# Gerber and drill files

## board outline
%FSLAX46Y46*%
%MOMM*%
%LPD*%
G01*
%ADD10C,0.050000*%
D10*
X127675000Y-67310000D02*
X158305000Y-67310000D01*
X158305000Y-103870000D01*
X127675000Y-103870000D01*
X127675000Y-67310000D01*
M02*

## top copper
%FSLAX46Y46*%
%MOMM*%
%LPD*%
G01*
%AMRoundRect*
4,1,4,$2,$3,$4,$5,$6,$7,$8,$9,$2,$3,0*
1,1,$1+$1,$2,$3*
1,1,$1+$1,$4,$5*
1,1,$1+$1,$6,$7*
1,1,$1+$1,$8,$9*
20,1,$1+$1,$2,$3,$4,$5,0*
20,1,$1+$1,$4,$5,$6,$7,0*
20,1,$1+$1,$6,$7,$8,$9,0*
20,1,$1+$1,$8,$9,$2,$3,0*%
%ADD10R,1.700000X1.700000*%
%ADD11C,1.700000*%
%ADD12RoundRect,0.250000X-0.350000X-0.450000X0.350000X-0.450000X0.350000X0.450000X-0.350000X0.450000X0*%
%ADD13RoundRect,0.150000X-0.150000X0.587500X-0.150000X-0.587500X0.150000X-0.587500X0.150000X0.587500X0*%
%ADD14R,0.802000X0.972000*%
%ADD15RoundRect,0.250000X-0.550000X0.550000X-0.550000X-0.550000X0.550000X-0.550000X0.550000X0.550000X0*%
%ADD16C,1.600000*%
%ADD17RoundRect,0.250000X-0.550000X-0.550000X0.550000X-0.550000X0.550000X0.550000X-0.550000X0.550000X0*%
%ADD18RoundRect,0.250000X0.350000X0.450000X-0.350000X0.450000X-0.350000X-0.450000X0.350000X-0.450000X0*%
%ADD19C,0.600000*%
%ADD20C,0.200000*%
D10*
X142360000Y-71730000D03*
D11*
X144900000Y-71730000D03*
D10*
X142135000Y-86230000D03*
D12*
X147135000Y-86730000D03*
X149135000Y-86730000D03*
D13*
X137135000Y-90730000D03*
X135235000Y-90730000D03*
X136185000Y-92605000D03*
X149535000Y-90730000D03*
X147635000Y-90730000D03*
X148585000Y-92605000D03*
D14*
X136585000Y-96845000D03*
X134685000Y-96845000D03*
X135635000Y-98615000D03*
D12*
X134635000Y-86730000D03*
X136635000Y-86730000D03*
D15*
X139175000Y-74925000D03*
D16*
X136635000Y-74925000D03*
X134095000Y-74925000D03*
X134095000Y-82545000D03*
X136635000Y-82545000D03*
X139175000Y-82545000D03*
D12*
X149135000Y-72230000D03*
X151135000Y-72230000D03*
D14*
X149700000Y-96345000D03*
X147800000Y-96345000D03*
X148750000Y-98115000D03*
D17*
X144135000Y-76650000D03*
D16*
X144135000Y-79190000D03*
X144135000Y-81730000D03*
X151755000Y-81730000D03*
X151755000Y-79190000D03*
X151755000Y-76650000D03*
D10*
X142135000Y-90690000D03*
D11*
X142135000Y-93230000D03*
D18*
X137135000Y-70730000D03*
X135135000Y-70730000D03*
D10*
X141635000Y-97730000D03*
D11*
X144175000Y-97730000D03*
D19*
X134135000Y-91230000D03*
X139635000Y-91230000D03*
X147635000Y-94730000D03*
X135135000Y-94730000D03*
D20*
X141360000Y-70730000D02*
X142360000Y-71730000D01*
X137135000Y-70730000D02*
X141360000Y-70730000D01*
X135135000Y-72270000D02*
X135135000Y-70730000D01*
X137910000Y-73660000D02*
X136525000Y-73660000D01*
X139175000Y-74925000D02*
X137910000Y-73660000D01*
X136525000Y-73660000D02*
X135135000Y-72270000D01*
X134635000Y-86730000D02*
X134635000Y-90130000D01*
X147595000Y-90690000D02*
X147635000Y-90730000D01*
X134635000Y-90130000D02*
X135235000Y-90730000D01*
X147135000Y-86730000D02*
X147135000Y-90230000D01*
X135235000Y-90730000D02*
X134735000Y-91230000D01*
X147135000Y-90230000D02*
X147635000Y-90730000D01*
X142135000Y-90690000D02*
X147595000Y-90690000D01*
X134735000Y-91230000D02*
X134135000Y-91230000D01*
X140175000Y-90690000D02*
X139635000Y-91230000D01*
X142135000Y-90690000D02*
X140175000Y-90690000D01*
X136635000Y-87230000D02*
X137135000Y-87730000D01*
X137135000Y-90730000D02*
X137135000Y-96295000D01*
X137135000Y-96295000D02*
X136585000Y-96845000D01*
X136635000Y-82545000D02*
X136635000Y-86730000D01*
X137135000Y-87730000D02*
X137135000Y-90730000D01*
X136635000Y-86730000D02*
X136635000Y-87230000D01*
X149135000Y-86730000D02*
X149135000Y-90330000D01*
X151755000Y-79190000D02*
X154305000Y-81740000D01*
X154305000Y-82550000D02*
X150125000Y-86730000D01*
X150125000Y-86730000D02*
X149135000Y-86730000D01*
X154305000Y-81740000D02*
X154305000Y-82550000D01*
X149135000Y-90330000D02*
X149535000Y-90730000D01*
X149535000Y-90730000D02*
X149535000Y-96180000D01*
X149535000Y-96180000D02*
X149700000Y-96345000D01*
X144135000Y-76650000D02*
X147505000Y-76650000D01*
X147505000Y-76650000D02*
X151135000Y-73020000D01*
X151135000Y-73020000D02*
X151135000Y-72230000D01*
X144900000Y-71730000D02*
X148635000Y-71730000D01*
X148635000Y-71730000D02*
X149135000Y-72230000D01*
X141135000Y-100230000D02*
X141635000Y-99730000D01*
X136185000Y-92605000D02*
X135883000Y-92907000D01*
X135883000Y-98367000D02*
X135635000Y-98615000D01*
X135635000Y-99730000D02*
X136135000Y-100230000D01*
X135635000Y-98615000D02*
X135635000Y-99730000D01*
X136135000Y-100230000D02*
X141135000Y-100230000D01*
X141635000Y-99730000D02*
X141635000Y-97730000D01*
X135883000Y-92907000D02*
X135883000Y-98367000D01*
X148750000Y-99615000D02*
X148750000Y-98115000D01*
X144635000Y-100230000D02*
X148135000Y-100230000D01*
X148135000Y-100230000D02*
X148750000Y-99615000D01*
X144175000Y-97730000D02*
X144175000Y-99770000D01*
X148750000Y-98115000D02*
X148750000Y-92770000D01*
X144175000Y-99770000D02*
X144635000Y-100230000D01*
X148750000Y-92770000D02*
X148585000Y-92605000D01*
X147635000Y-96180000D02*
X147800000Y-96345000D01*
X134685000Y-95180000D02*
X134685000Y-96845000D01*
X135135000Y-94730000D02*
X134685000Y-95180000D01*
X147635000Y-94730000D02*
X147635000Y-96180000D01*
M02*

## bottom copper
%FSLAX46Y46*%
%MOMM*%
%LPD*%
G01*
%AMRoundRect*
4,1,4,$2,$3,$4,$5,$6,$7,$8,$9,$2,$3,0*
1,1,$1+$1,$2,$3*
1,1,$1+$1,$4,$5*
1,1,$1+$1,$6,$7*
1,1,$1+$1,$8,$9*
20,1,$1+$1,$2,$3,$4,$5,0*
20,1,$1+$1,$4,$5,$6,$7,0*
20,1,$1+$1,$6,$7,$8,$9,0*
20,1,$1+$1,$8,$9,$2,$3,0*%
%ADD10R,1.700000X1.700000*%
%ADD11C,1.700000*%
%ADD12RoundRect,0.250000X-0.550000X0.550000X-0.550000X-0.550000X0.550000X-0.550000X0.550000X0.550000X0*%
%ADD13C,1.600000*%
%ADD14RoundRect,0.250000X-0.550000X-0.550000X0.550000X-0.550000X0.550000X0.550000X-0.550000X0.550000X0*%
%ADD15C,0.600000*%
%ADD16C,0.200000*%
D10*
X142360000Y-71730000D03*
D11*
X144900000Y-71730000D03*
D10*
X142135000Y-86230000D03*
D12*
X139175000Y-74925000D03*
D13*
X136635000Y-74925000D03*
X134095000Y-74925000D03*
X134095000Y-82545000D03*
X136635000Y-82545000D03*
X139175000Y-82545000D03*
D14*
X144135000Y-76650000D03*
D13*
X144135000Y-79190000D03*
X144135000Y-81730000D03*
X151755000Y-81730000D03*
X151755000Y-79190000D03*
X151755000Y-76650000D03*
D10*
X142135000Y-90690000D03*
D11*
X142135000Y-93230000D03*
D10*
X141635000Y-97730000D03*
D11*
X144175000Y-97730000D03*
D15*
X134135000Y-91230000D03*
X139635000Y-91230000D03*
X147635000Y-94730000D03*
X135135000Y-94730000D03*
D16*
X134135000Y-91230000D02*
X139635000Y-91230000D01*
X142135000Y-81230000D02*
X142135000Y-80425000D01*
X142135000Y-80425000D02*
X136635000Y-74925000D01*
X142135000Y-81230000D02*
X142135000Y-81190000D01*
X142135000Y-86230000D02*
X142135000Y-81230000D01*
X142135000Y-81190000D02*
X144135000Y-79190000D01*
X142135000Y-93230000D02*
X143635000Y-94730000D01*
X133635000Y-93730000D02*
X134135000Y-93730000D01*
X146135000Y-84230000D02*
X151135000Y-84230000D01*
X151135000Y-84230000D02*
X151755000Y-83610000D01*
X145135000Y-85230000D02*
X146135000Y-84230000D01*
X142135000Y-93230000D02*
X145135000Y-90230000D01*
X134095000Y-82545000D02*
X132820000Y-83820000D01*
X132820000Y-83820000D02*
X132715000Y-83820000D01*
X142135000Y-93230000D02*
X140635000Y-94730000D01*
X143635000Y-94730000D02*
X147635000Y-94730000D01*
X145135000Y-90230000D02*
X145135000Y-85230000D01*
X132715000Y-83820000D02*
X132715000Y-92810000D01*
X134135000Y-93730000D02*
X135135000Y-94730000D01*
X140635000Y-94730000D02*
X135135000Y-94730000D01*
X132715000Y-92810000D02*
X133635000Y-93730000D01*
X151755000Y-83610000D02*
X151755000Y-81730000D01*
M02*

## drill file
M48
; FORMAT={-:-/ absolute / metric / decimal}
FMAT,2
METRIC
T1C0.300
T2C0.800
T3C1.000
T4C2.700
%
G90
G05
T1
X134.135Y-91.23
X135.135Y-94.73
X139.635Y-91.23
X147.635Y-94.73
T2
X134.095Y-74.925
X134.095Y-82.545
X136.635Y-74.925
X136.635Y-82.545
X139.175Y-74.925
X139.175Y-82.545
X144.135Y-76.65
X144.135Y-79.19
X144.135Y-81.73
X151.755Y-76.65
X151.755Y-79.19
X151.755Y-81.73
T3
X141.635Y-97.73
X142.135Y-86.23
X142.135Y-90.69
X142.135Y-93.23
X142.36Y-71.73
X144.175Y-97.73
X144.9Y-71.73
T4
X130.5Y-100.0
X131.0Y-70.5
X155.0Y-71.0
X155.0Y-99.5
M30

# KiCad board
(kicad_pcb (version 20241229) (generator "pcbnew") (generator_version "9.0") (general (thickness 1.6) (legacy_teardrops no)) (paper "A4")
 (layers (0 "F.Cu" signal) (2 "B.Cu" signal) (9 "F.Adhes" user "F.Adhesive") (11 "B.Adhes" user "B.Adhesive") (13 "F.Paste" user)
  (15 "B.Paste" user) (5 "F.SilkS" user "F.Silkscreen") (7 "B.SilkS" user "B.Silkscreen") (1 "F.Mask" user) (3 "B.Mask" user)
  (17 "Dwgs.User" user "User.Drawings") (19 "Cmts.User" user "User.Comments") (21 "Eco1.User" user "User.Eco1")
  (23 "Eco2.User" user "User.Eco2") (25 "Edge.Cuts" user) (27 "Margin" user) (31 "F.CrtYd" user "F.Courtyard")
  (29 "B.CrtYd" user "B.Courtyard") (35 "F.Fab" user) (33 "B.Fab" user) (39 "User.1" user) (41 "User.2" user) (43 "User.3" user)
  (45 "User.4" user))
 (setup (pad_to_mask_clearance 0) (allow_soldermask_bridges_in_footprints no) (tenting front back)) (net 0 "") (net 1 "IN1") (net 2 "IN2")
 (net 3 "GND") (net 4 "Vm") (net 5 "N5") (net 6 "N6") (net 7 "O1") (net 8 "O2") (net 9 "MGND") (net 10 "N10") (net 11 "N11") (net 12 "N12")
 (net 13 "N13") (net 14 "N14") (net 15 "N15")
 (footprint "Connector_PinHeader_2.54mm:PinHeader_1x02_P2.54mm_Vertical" (layer "F.Cu") (at 142.36 71.73 90)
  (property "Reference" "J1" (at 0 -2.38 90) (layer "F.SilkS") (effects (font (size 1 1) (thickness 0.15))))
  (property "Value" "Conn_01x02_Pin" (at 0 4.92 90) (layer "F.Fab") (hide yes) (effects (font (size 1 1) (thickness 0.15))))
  (pad "1" thru_hole rect (at 0 0 90) (size 1.7 1.7) (drill 1) (layers "*.Cu" "*.Mask") (remove_unused_layers no) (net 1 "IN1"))
  (pad "2" thru_hole circle (at 0 2.54 90) (size 1.7 1.7) (drill 1) (layers "*.Cu" "*.Mask") (remove_unused_layers no) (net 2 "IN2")))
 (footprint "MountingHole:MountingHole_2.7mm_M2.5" (layer "F.Cu") (at 155 71)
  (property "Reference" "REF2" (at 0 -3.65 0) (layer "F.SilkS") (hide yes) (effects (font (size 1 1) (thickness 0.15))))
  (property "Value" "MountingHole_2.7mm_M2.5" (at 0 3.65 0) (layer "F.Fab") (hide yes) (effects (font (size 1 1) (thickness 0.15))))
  (pad "" np_thru_hole circle (at 0 0) (size 2.7 2.7) (drill 2.7) (layers "*.Cu" "*.Mask")))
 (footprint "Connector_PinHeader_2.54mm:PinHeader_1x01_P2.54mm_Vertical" (layer "F.Cu") (at 142.135 86.23)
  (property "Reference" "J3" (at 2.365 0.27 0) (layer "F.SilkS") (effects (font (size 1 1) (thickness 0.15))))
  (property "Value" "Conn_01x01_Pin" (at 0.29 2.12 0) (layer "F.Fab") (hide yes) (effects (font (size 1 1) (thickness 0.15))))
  (pad "1" thru_hole rect (at 0 0) (size 1.7 1.7) (drill 1) (layers "*.Cu" "*.Mask") (remove_unused_layers no) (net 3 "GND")))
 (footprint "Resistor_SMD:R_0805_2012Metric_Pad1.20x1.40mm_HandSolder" (layer "F.Cu") (at 148.135 86.73)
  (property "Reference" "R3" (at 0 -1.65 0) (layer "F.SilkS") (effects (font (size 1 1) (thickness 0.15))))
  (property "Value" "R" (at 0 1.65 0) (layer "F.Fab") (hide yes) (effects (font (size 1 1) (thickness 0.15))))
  (pad "1" smd roundrect (at -1 0) (size 1.2 1.4) (layers "F.Cu" "F.Mask" "F.Paste") (roundrect_rratio 0.208333) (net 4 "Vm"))
  (pad "2" smd roundrect (at 1 0) (size 1.2 1.4) (layers "F.Cu" "F.Mask" "F.Paste") (roundrect_rratio 0.208333) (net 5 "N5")))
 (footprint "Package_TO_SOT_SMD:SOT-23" (layer "F.Cu") (at 136.185 91.6675 -90)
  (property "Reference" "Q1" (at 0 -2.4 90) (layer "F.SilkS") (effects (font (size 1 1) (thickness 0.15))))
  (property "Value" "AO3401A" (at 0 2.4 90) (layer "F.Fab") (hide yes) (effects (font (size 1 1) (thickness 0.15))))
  (pad "1" smd roundrect (at -0.9375 -0.95 270) (size 1.475 0.6) (layers "F.Cu" "F.Mask" "F.Paste") (roundrect_rratio 0.25) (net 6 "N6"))
  (pad "2" smd roundrect (at -0.9375 0.95 270) (size 1.475 0.6) (layers "F.Cu" "F.Mask" "F.Paste") (roundrect_rratio 0.25) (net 4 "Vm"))
  (pad "3" smd roundrect (at 0.9375 0 270) (size 1.475 0.6) (layers "F.Cu" "F.Mask" "F.Paste") (roundrect_rratio 0.25) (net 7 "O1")))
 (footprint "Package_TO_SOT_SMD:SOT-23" (layer "F.Cu") (at 148.585 91.6675 -90)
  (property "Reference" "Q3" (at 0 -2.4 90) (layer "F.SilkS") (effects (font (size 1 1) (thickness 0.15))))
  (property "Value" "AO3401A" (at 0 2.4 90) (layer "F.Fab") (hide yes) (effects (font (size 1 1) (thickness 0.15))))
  (pad "1" smd roundrect (at -0.9375 -0.95 270) (size 1.475 0.6) (layers "F.Cu" "F.Mask" "F.Paste") (roundrect_rratio 0.25) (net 5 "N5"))
  (pad "2" smd roundrect (at -0.9375 0.95 270) (size 1.475 0.6) (layers "F.Cu" "F.Mask" "F.Paste") (roundrect_rratio 0.25) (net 4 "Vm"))
  (pad "3" smd roundrect (at 0.9375 0 270) (size 1.475 0.6) (layers "F.Cu" "F.Mask" "F.Paste") (roundrect_rratio 0.25) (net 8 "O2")))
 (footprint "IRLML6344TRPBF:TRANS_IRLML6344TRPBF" (layer "F.Cu") (at 135.635 97.73 -90)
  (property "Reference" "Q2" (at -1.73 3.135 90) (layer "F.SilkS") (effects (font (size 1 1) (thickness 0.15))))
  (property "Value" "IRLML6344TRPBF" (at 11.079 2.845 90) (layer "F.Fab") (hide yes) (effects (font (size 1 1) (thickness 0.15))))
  (pad "1" smd rect (at -0.885 -0.95 270) (size 0.972 0.802) (layers "F.Cu" "F.Mask" "F.Paste") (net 6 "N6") (solder_mask_margin 0.102))
  (pad "2" smd rect (at -0.885 0.95 270) (size 0.972 0.802) (layers "F.Cu" "F.Mask" "F.Paste") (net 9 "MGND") (solder_mask_margin 0.102))
  (pad "3" smd rect (at 0.885 0 270) (size 0.972 0.802) (layers "F.Cu" "F.Mask" "F.Paste") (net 7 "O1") (solder_mask_margin 0.102)))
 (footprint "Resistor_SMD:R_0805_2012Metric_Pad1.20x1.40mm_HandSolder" (layer "F.Cu") (at 135.635 86.73)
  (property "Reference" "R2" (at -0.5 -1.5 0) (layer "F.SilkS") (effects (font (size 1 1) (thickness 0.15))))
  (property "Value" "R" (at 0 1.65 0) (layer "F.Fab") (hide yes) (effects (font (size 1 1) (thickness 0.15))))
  (pad "1" smd roundrect (at -1 0) (size 1.2 1.4) (layers "F.Cu" "F.Mask" "F.Paste") (roundrect_rratio 0.208333) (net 4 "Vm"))
  (pad "2" smd roundrect (at 1 0) (size 1.2 1.4) (layers "F.Cu" "F.Mask" "F.Paste") (roundrect_rratio 0.208333) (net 6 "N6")))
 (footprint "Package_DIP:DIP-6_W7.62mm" (layer "F.Cu") (at 139.175 74.925 -90)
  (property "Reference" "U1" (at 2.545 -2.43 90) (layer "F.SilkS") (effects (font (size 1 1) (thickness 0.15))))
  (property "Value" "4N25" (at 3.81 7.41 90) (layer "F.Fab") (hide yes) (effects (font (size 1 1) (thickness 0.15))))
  (pad "1" thru_hole roundrect (at 0 0 270) (size 1.6 1.6) (drill 0.8) (layers "*.Cu" "*.Mask") (remove_unused_layers no)
   (roundrect_rratio 0.15625) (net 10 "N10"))
  (pad "2" thru_hole circle (at 0 2.54 270) (size 1.6 1.6) (drill 0.8) (layers "*.Cu" "*.Mask") (remove_unused_layers no) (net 3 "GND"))
  (pad "3" thru_hole circle (at 0 5.08 270) (size 1.6 1.6) (drill 0.8) (layers "*.Cu" "*.Mask") (remove_unused_layers no) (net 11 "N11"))
  (pad "4" thru_hole circle (at 7.62 5.08 270) (size 1.6 1.6) (drill 0.8) (layers "*.Cu" "*.Mask") (remove_unused_layers no) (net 9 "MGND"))
  (pad "5" thru_hole circle (at 7.62 2.54 270) (size 1.6 1.6) (drill 0.8) (layers "*.Cu" "*.Mask") (remove_unused_layers no) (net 6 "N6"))
  (pad "6" thru_hole circle (at 7.62 0 270) (size 1.6 1.6) (drill 0.8) (layers "*.Cu" "*.Mask") (remove_unused_layers no) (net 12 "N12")))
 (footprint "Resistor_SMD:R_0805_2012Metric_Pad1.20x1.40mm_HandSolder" (layer "F.Cu") (at 150.135 72.23)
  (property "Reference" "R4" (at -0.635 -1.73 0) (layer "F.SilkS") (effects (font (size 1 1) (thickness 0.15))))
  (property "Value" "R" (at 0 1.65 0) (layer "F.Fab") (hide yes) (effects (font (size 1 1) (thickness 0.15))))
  (pad "1" smd roundrect (at -1 0) (size 1.2 1.4) (layers "F.Cu" "F.Mask" "F.Paste") (roundrect_rratio 0.208333) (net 2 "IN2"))
  (pad "2" smd roundrect (at 1 0) (size 1.2 1.4) (layers "F.Cu" "F.Mask" "F.Paste") (roundrect_rratio 0.208333) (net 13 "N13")))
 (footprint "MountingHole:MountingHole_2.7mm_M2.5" (layer "F.Cu") (at 130.5 100)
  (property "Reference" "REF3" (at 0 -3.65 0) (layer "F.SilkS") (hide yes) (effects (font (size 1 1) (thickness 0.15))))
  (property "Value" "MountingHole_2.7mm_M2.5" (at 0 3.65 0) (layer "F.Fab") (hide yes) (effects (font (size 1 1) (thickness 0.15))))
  (pad "" np_thru_hole circle (at 0 0) (size 2.7 2.7) (drill 2.7) (layers "*.Cu" "*.Mask")))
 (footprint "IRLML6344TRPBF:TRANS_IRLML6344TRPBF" (layer "F.Cu") (at 148.75 97.23 -90)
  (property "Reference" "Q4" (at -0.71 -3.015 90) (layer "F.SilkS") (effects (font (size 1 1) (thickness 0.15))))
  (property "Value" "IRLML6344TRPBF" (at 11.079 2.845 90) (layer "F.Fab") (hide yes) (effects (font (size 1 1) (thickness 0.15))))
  (pad "1" smd rect (at -0.885 -0.95 270) (size 0.972 0.802) (layers "F.Cu" "F.Mask" "F.Paste") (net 5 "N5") (solder_mask_margin 0.102))
  (pad "2" smd rect (at -0.885 0.95 270) (size 0.972 0.802) (layers "F.Cu" "F.Mask" "F.Paste") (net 9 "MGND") (solder_mask_margin 0.102))
  (pad "3" smd rect (at 0.885 0 270) (size 0.972 0.802) (layers "F.Cu" "F.Mask" "F.Paste") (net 8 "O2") (solder_mask_margin 0.102)))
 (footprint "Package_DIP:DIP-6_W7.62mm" (layer "F.Cu") (at 144.135 76.65)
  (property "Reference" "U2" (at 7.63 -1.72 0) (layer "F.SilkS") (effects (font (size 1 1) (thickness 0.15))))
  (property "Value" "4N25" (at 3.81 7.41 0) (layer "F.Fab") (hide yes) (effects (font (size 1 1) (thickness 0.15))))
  (pad "1" thru_hole roundrect (at 0 0) (size 1.6 1.6) (drill 0.8) (layers "*.Cu" "*.Mask") (remove_unused_layers no)
   (roundrect_rratio 0.15625) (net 13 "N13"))
  (pad "2" thru_hole circle (at 0 2.54) (size 1.6 1.6) (drill 0.8) (layers "*.Cu" "*.Mask") (remove_unused_layers no) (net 3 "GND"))
  (pad "3" thru_hole circle (at 0 5.08) (size 1.6 1.6) (drill 0.8) (layers "*.Cu" "*.Mask") (remove_unused_layers no) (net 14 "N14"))
  (pad "4" thru_hole circle (at 7.62 5.08) (size 1.6 1.6) (drill 0.8) (layers "*.Cu" "*.Mask") (remove_unused_layers no) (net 9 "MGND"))
  (pad "5" thru_hole circle (at 7.62 2.54) (size 1.6 1.6) (drill 0.8) (layers "*.Cu" "*.Mask") (remove_unused_layers no) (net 5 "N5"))
  (pad "6" thru_hole circle (at 7.62 0) (size 1.6 1.6) (drill 0.8) (layers "*.Cu" "*.Mask") (remove_unused_layers no) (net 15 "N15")))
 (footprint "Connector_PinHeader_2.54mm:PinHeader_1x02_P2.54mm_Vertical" (layer "F.Cu") (at 142.135 90.69)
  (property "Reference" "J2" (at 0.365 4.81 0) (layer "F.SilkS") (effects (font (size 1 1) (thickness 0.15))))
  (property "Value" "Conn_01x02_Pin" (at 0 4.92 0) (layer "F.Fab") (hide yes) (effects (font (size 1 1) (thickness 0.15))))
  (pad "1" thru_hole rect (at 0 0) (size 1.7 1.7) (drill 1) (layers "*.Cu" "*.Mask") (remove_unused_layers no) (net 4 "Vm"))
  (pad "2" thru_hole circle (at 0 2.54) (size 1.7 1.7) (drill 1) (layers "*.Cu" "*.Mask") (remove_unused_layers no) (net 9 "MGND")))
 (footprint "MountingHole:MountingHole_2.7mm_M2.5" (layer "F.Cu") (at 131 70.5)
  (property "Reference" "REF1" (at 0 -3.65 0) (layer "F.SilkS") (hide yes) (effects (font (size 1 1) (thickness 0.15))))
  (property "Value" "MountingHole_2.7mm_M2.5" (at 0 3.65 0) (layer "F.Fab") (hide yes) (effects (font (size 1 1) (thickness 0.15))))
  (pad "" np_thru_hole circle (at 0 0) (size 2.7 2.7) (drill 2.7) (layers "*.Cu" "*.Mask")))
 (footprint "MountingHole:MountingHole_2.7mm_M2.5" (layer "F.Cu") (at 155 99.5)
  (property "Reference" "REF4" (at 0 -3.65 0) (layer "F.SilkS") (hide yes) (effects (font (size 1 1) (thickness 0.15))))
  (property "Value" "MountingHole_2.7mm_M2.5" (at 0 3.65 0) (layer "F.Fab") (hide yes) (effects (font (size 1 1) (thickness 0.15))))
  (pad "" np_thru_hole circle (at 0 0) (size 2.7 2.7) (drill 2.7) (layers "*.Cu" "*.Mask")))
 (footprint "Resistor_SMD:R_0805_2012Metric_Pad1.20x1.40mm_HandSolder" (layer "F.Cu") (at 136.135 70.73 180)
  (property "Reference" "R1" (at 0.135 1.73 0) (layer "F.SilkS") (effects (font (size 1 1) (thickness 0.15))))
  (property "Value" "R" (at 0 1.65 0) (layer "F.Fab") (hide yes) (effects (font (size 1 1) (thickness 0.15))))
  (pad "1" smd roundrect (at -1 0 180) (size 1.2 1.4) (layers "F.Cu" "F.Mask" "F.Paste") (roundrect_rratio 0.208333) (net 1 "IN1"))
  (pad "2" smd roundrect (at 1 0 180) (size 1.2 1.4) (layers "F.Cu" "F.Mask" "F.Paste") (roundrect_rratio 0.208333) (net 10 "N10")))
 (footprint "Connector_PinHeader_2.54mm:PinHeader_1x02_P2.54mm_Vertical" (layer "F.Cu") (at 141.635 97.73 90)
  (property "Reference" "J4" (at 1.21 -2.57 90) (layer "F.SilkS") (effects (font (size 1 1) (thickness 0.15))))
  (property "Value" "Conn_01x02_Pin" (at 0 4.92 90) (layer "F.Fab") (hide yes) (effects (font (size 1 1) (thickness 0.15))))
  (pad "1" thru_hole rect (at 0 0 90) (size 1.7 1.7) (drill 1) (layers "*.Cu" "*.Mask") (remove_unused_layers no) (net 7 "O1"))
  (pad "2" thru_hole circle (at 0 2.54 90) (size 1.7 1.7) (drill 1) (layers "*.Cu" "*.Mask") (remove_unused_layers no) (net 8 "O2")))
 (gr_rect (start 127.675 67.31) (end 158.305 103.87) (stroke (width 0.05) (type default)) (fill no) (layer "Edge.Cuts"))
 (segment (start 141.36 70.73) (end 142.36 71.73) (width 0.2) (layer "F.Cu") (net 1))
 (segment (start 137.135 70.73) (end 141.36 70.73) (width 0.2) (layer "F.Cu") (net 1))
 (segment (start 135.135 72.27) (end 135.135 70.73) (width 0.2) (layer "F.Cu") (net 10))
 (segment (start 137.91 73.66) (end 136.525 73.66) (width 0.2) (layer "F.Cu") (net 10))
 (segment (start 139.175 74.925) (end 137.91 73.66) (width 0.2) (layer "F.Cu") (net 10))
 (segment (start 136.525 73.66) (end 135.135 72.27) (width 0.2) (layer "F.Cu") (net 10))
 (segment (start 134.635 86.73) (end 134.635 90.13) (width 0.2) (layer "F.Cu") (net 4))
 (segment (start 147.595 90.69) (end 147.635 90.73) (width 0.2) (layer "F.Cu") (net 4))
 (segment (start 134.635 90.13) (end 135.235 90.73) (width 0.2) (layer "F.Cu") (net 4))
 (segment (start 147.135 86.73) (end 147.135 90.23) (width 0.2) (layer "F.Cu") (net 4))
 (segment (start 135.235 90.73) (end 134.735 91.23) (width 0.2) (layer "F.Cu") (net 4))
 (segment (start 147.135 90.23) (end 147.635 90.73) (width 0.2) (layer "F.Cu") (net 4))
 (segment (start 142.135 90.69) (end 147.595 90.69) (width 0.2) (layer "F.Cu") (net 4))
 (segment (start 134.735 91.23) (end 134.135 91.23) (width 0.2) (layer "F.Cu") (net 4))
 (segment (start 140.175 90.69) (end 139.635 91.23) (width 0.2) (layer "F.Cu") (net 4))
 (segment (start 142.135 90.69) (end 140.175 90.69) (width 0.2) (layer "F.Cu") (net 4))
 (via (at 134.135 91.23) (size 0.6) (drill 0.3) (layers "F.Cu" "B.Cu") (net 4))
 (via (at 139.635 91.23) (size 0.6) (drill 0.3) (layers "F.Cu" "B.Cu") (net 4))
 (segment (start 134.135 91.23) (end 139.635 91.23) (width 0.2) (layer "B.Cu") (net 4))
 (segment (start 136.635 87.23) (end 137.135 87.73) (width 0.2) (layer "F.Cu") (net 6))
 (segment (start 137.135 90.73) (end 137.135 96.295) (width 0.2) (layer "F.Cu") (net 6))
 (segment (start 137.135 96.295) (end 136.585 96.845) (width 0.2) (layer "F.Cu") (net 6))
 (segment (start 136.635 82.545) (end 136.635 86.73) (width 0.2) (layer "F.Cu") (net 6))
 (segment (start 137.135 87.73) (end 137.135 90.73) (width 0.2) (layer "F.Cu") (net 6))
 (segment (start 136.635 86.73) (end 136.635 87.23) (width 0.2) (layer "F.Cu") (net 6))
 (segment (start 149.135 86.73) (end 149.135 90.33) (width 0.2) (layer "F.Cu") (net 5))
 (segment (start 151.755 79.19) (end 154.305 81.74) (width 0.2) (layer "F.Cu") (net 5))
 (segment (start 154.305 82.55) (end 150.125 86.73) (width 0.2) (layer "F.Cu") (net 5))
 (segment (start 150.125 86.73) (end 149.135 86.73) (width 0.2) (layer "F.Cu") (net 5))
 (segment (start 154.305 81.74) (end 154.305 82.55) (width 0.2) (layer "F.Cu") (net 5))
 (segment (start 149.135 90.33) (end 149.535 90.73) (width 0.2) (layer "F.Cu") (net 5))
 (segment (start 149.535 90.73) (end 149.535 96.18) (width 0.2) (layer "F.Cu") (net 5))
 (segment (start 149.535 96.18) (end 149.7 96.345) (width 0.2) (layer "F.Cu") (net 5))
 (segment (start 144.135 76.65) (end 147.505 76.65) (width 0.2) (layer "F.Cu") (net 13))
 (segment (start 147.505 76.65) (end 151.135 73.02) (width 0.2) (layer "F.Cu") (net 13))
 (segment (start 151.135 73.02) (end 151.135 72.23) (width 0.2) (layer "F.Cu") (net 13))
 (segment (start 144.9 71.73) (end 148.635 71.73) (width 0.2) (layer "F.Cu") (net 2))
 (segment (start 148.635 71.73) (end 149.135 72.23) (width 0.2) (layer "F.Cu") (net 2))
 (segment (start 141.135 100.23) (end 141.635 99.73) (width 0.2) (layer "F.Cu") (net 7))
 (segment (start 136.185 92.605) (end 135.883 92.907) (width 0.2) (layer "F.Cu") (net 7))
 (segment (start 135.883 98.367) (end 135.635 98.615) (width 0.2) (layer "F.Cu") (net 7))
 (segment (start 135.635 99.73) (end 136.135 100.23) (width 0.2) (layer "F.Cu") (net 7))
 (segment (start 135.635 98.615) (end 135.635 99.73) (width 0.2) (layer "F.Cu") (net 7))
 (segment (start 136.135 100.23) (end 141.135 100.23) (width 0.2) (layer "F.Cu") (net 7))
 (segment (start 141.635 99.73) (end 141.635 97.73) (width 0.2) (layer "F.Cu") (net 7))
 (segment (start 135.883 92.907) (end 135.883 98.367) (width 0.2) (layer "F.Cu") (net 7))
 (segment (start 148.75 99.615) (end 148.75 98.115) (width 0.2) (layer "F.Cu") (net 8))
 (segment (start 144.635 100.23) (end 148.135 100.23) (width 0.2) (layer "F.Cu") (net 8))
 (segment (start 148.135 100.23) (end 148.75 99.615) (width 0.2) (layer "F.Cu") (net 8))
 (segment (start 144.175 97.73) (end 144.175 99.77) (width 0.2) (layer "F.Cu") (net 8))
 (segment (start 148.75 98.115) (end 148.75 92.77) (width 0.2) (layer "F.Cu") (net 8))
 (segment (start 144.175 99.77) (end 144.635 100.23) (width 0.2) (layer "F.Cu") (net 8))
 (segment (start 148.75 92.77) (end 148.585 92.605) (width 0.2) (layer "F.Cu") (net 8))
 (segment (start 142.135 81.23) (end 142.135 80.425) (width 0.2) (layer "B.Cu") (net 3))
 (segment (start 142.135 80.425) (end 136.635 74.925) (width 0.2) (layer "B.Cu") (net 3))
 (segment (start 142.135 81.23) (end 142.135 81.19) (width 0.2) (layer "B.Cu") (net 3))
 (segment (start 142.135 86.23) (end 142.135 81.23) (width 0.2) (layer "B.Cu") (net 3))
 (segment (start 142.135 81.19) (end 144.135 79.19) (width 0.2) (layer "B.Cu") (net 3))
 (segment (start 147.635 96.18) (end 147.8 96.345) (width 0.2) (layer "F.Cu") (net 9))
 (segment (start 134.685 95.18) (end 134.685 96.845) (width 0.2) (layer "F.Cu") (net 9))
 (segment (start 135.135 94.73) (end 134.685 95.18) (width 0.2) (layer "F.Cu") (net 9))
 (segment (start 147.635 94.73) (end 147.635 96.18) (width 0.2) (layer "F.Cu") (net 9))
 (via (at 147.635 94.73) (size 0.6) (drill 0.3) (layers "F.Cu" "B.Cu") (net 9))
 (via (at 135.135 94.73) (size 0.6) (drill 0.3) (layers "F.Cu" "B.Cu") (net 9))
 (segment (start 142.135 93.23) (end 143.635 94.73) (width 0.2) (layer "B.Cu") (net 9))
 (segment (start 133.635 93.73) (end 134.135 93.73) (width 0.2) (layer "B.Cu") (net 9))
 (segment (start 146.135 84.23) (end 151.135 84.23) (width 0.2) (layer "B.Cu") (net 9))
 (segment (start 151.135 84.23) (end 151.755 83.61) (width 0.2) (layer "B.Cu") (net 9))
 (segment (start 145.135 85.23) (end 146.135 84.23) (width 0.2) (layer "B.Cu") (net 9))
 (segment (start 142.135 93.23) (end 145.135 90.23) (width 0.2) (layer "B.Cu") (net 9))
 (segment (start 134.095 82.545) (end 132.82 83.82) (width 0.2) (layer "B.Cu") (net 9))
 (segment (start 132.82 83.82) (end 132.715 83.82) (width 0.2) (layer "B.Cu") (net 9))
 (segment (start 142.135 93.23) (end 140.635 94.73) (width 0.2) (layer "B.Cu") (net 9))
 (segment (start 143.635 94.73) (end 147.635 94.73) (width 0.2) (layer "B.Cu") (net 9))
 (segment (start 145.135 90.23) (end 145.135 85.23) (width 0.2) (layer "B.Cu") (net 9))
 (segment (start 132.715 83.82) (end 132.715 92.81) (width 0.2) (layer "B.Cu") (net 9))
 (segment (start 134.135 93.73) (end 135.135 94.73) (width 0.2) (layer "B.Cu") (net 9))
 (segment (start 140.635 94.73) (end 135.135 94.73) (width 0.2) (layer "B.Cu") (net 9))
 (segment (start 132.715 92.81) (end 133.635 93.73) (width 0.2) (layer "B.Cu") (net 9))
 (segment (start 151.755 83.61) (end 151.755 81.73) (width 0.2) (layer "B.Cu") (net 9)))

